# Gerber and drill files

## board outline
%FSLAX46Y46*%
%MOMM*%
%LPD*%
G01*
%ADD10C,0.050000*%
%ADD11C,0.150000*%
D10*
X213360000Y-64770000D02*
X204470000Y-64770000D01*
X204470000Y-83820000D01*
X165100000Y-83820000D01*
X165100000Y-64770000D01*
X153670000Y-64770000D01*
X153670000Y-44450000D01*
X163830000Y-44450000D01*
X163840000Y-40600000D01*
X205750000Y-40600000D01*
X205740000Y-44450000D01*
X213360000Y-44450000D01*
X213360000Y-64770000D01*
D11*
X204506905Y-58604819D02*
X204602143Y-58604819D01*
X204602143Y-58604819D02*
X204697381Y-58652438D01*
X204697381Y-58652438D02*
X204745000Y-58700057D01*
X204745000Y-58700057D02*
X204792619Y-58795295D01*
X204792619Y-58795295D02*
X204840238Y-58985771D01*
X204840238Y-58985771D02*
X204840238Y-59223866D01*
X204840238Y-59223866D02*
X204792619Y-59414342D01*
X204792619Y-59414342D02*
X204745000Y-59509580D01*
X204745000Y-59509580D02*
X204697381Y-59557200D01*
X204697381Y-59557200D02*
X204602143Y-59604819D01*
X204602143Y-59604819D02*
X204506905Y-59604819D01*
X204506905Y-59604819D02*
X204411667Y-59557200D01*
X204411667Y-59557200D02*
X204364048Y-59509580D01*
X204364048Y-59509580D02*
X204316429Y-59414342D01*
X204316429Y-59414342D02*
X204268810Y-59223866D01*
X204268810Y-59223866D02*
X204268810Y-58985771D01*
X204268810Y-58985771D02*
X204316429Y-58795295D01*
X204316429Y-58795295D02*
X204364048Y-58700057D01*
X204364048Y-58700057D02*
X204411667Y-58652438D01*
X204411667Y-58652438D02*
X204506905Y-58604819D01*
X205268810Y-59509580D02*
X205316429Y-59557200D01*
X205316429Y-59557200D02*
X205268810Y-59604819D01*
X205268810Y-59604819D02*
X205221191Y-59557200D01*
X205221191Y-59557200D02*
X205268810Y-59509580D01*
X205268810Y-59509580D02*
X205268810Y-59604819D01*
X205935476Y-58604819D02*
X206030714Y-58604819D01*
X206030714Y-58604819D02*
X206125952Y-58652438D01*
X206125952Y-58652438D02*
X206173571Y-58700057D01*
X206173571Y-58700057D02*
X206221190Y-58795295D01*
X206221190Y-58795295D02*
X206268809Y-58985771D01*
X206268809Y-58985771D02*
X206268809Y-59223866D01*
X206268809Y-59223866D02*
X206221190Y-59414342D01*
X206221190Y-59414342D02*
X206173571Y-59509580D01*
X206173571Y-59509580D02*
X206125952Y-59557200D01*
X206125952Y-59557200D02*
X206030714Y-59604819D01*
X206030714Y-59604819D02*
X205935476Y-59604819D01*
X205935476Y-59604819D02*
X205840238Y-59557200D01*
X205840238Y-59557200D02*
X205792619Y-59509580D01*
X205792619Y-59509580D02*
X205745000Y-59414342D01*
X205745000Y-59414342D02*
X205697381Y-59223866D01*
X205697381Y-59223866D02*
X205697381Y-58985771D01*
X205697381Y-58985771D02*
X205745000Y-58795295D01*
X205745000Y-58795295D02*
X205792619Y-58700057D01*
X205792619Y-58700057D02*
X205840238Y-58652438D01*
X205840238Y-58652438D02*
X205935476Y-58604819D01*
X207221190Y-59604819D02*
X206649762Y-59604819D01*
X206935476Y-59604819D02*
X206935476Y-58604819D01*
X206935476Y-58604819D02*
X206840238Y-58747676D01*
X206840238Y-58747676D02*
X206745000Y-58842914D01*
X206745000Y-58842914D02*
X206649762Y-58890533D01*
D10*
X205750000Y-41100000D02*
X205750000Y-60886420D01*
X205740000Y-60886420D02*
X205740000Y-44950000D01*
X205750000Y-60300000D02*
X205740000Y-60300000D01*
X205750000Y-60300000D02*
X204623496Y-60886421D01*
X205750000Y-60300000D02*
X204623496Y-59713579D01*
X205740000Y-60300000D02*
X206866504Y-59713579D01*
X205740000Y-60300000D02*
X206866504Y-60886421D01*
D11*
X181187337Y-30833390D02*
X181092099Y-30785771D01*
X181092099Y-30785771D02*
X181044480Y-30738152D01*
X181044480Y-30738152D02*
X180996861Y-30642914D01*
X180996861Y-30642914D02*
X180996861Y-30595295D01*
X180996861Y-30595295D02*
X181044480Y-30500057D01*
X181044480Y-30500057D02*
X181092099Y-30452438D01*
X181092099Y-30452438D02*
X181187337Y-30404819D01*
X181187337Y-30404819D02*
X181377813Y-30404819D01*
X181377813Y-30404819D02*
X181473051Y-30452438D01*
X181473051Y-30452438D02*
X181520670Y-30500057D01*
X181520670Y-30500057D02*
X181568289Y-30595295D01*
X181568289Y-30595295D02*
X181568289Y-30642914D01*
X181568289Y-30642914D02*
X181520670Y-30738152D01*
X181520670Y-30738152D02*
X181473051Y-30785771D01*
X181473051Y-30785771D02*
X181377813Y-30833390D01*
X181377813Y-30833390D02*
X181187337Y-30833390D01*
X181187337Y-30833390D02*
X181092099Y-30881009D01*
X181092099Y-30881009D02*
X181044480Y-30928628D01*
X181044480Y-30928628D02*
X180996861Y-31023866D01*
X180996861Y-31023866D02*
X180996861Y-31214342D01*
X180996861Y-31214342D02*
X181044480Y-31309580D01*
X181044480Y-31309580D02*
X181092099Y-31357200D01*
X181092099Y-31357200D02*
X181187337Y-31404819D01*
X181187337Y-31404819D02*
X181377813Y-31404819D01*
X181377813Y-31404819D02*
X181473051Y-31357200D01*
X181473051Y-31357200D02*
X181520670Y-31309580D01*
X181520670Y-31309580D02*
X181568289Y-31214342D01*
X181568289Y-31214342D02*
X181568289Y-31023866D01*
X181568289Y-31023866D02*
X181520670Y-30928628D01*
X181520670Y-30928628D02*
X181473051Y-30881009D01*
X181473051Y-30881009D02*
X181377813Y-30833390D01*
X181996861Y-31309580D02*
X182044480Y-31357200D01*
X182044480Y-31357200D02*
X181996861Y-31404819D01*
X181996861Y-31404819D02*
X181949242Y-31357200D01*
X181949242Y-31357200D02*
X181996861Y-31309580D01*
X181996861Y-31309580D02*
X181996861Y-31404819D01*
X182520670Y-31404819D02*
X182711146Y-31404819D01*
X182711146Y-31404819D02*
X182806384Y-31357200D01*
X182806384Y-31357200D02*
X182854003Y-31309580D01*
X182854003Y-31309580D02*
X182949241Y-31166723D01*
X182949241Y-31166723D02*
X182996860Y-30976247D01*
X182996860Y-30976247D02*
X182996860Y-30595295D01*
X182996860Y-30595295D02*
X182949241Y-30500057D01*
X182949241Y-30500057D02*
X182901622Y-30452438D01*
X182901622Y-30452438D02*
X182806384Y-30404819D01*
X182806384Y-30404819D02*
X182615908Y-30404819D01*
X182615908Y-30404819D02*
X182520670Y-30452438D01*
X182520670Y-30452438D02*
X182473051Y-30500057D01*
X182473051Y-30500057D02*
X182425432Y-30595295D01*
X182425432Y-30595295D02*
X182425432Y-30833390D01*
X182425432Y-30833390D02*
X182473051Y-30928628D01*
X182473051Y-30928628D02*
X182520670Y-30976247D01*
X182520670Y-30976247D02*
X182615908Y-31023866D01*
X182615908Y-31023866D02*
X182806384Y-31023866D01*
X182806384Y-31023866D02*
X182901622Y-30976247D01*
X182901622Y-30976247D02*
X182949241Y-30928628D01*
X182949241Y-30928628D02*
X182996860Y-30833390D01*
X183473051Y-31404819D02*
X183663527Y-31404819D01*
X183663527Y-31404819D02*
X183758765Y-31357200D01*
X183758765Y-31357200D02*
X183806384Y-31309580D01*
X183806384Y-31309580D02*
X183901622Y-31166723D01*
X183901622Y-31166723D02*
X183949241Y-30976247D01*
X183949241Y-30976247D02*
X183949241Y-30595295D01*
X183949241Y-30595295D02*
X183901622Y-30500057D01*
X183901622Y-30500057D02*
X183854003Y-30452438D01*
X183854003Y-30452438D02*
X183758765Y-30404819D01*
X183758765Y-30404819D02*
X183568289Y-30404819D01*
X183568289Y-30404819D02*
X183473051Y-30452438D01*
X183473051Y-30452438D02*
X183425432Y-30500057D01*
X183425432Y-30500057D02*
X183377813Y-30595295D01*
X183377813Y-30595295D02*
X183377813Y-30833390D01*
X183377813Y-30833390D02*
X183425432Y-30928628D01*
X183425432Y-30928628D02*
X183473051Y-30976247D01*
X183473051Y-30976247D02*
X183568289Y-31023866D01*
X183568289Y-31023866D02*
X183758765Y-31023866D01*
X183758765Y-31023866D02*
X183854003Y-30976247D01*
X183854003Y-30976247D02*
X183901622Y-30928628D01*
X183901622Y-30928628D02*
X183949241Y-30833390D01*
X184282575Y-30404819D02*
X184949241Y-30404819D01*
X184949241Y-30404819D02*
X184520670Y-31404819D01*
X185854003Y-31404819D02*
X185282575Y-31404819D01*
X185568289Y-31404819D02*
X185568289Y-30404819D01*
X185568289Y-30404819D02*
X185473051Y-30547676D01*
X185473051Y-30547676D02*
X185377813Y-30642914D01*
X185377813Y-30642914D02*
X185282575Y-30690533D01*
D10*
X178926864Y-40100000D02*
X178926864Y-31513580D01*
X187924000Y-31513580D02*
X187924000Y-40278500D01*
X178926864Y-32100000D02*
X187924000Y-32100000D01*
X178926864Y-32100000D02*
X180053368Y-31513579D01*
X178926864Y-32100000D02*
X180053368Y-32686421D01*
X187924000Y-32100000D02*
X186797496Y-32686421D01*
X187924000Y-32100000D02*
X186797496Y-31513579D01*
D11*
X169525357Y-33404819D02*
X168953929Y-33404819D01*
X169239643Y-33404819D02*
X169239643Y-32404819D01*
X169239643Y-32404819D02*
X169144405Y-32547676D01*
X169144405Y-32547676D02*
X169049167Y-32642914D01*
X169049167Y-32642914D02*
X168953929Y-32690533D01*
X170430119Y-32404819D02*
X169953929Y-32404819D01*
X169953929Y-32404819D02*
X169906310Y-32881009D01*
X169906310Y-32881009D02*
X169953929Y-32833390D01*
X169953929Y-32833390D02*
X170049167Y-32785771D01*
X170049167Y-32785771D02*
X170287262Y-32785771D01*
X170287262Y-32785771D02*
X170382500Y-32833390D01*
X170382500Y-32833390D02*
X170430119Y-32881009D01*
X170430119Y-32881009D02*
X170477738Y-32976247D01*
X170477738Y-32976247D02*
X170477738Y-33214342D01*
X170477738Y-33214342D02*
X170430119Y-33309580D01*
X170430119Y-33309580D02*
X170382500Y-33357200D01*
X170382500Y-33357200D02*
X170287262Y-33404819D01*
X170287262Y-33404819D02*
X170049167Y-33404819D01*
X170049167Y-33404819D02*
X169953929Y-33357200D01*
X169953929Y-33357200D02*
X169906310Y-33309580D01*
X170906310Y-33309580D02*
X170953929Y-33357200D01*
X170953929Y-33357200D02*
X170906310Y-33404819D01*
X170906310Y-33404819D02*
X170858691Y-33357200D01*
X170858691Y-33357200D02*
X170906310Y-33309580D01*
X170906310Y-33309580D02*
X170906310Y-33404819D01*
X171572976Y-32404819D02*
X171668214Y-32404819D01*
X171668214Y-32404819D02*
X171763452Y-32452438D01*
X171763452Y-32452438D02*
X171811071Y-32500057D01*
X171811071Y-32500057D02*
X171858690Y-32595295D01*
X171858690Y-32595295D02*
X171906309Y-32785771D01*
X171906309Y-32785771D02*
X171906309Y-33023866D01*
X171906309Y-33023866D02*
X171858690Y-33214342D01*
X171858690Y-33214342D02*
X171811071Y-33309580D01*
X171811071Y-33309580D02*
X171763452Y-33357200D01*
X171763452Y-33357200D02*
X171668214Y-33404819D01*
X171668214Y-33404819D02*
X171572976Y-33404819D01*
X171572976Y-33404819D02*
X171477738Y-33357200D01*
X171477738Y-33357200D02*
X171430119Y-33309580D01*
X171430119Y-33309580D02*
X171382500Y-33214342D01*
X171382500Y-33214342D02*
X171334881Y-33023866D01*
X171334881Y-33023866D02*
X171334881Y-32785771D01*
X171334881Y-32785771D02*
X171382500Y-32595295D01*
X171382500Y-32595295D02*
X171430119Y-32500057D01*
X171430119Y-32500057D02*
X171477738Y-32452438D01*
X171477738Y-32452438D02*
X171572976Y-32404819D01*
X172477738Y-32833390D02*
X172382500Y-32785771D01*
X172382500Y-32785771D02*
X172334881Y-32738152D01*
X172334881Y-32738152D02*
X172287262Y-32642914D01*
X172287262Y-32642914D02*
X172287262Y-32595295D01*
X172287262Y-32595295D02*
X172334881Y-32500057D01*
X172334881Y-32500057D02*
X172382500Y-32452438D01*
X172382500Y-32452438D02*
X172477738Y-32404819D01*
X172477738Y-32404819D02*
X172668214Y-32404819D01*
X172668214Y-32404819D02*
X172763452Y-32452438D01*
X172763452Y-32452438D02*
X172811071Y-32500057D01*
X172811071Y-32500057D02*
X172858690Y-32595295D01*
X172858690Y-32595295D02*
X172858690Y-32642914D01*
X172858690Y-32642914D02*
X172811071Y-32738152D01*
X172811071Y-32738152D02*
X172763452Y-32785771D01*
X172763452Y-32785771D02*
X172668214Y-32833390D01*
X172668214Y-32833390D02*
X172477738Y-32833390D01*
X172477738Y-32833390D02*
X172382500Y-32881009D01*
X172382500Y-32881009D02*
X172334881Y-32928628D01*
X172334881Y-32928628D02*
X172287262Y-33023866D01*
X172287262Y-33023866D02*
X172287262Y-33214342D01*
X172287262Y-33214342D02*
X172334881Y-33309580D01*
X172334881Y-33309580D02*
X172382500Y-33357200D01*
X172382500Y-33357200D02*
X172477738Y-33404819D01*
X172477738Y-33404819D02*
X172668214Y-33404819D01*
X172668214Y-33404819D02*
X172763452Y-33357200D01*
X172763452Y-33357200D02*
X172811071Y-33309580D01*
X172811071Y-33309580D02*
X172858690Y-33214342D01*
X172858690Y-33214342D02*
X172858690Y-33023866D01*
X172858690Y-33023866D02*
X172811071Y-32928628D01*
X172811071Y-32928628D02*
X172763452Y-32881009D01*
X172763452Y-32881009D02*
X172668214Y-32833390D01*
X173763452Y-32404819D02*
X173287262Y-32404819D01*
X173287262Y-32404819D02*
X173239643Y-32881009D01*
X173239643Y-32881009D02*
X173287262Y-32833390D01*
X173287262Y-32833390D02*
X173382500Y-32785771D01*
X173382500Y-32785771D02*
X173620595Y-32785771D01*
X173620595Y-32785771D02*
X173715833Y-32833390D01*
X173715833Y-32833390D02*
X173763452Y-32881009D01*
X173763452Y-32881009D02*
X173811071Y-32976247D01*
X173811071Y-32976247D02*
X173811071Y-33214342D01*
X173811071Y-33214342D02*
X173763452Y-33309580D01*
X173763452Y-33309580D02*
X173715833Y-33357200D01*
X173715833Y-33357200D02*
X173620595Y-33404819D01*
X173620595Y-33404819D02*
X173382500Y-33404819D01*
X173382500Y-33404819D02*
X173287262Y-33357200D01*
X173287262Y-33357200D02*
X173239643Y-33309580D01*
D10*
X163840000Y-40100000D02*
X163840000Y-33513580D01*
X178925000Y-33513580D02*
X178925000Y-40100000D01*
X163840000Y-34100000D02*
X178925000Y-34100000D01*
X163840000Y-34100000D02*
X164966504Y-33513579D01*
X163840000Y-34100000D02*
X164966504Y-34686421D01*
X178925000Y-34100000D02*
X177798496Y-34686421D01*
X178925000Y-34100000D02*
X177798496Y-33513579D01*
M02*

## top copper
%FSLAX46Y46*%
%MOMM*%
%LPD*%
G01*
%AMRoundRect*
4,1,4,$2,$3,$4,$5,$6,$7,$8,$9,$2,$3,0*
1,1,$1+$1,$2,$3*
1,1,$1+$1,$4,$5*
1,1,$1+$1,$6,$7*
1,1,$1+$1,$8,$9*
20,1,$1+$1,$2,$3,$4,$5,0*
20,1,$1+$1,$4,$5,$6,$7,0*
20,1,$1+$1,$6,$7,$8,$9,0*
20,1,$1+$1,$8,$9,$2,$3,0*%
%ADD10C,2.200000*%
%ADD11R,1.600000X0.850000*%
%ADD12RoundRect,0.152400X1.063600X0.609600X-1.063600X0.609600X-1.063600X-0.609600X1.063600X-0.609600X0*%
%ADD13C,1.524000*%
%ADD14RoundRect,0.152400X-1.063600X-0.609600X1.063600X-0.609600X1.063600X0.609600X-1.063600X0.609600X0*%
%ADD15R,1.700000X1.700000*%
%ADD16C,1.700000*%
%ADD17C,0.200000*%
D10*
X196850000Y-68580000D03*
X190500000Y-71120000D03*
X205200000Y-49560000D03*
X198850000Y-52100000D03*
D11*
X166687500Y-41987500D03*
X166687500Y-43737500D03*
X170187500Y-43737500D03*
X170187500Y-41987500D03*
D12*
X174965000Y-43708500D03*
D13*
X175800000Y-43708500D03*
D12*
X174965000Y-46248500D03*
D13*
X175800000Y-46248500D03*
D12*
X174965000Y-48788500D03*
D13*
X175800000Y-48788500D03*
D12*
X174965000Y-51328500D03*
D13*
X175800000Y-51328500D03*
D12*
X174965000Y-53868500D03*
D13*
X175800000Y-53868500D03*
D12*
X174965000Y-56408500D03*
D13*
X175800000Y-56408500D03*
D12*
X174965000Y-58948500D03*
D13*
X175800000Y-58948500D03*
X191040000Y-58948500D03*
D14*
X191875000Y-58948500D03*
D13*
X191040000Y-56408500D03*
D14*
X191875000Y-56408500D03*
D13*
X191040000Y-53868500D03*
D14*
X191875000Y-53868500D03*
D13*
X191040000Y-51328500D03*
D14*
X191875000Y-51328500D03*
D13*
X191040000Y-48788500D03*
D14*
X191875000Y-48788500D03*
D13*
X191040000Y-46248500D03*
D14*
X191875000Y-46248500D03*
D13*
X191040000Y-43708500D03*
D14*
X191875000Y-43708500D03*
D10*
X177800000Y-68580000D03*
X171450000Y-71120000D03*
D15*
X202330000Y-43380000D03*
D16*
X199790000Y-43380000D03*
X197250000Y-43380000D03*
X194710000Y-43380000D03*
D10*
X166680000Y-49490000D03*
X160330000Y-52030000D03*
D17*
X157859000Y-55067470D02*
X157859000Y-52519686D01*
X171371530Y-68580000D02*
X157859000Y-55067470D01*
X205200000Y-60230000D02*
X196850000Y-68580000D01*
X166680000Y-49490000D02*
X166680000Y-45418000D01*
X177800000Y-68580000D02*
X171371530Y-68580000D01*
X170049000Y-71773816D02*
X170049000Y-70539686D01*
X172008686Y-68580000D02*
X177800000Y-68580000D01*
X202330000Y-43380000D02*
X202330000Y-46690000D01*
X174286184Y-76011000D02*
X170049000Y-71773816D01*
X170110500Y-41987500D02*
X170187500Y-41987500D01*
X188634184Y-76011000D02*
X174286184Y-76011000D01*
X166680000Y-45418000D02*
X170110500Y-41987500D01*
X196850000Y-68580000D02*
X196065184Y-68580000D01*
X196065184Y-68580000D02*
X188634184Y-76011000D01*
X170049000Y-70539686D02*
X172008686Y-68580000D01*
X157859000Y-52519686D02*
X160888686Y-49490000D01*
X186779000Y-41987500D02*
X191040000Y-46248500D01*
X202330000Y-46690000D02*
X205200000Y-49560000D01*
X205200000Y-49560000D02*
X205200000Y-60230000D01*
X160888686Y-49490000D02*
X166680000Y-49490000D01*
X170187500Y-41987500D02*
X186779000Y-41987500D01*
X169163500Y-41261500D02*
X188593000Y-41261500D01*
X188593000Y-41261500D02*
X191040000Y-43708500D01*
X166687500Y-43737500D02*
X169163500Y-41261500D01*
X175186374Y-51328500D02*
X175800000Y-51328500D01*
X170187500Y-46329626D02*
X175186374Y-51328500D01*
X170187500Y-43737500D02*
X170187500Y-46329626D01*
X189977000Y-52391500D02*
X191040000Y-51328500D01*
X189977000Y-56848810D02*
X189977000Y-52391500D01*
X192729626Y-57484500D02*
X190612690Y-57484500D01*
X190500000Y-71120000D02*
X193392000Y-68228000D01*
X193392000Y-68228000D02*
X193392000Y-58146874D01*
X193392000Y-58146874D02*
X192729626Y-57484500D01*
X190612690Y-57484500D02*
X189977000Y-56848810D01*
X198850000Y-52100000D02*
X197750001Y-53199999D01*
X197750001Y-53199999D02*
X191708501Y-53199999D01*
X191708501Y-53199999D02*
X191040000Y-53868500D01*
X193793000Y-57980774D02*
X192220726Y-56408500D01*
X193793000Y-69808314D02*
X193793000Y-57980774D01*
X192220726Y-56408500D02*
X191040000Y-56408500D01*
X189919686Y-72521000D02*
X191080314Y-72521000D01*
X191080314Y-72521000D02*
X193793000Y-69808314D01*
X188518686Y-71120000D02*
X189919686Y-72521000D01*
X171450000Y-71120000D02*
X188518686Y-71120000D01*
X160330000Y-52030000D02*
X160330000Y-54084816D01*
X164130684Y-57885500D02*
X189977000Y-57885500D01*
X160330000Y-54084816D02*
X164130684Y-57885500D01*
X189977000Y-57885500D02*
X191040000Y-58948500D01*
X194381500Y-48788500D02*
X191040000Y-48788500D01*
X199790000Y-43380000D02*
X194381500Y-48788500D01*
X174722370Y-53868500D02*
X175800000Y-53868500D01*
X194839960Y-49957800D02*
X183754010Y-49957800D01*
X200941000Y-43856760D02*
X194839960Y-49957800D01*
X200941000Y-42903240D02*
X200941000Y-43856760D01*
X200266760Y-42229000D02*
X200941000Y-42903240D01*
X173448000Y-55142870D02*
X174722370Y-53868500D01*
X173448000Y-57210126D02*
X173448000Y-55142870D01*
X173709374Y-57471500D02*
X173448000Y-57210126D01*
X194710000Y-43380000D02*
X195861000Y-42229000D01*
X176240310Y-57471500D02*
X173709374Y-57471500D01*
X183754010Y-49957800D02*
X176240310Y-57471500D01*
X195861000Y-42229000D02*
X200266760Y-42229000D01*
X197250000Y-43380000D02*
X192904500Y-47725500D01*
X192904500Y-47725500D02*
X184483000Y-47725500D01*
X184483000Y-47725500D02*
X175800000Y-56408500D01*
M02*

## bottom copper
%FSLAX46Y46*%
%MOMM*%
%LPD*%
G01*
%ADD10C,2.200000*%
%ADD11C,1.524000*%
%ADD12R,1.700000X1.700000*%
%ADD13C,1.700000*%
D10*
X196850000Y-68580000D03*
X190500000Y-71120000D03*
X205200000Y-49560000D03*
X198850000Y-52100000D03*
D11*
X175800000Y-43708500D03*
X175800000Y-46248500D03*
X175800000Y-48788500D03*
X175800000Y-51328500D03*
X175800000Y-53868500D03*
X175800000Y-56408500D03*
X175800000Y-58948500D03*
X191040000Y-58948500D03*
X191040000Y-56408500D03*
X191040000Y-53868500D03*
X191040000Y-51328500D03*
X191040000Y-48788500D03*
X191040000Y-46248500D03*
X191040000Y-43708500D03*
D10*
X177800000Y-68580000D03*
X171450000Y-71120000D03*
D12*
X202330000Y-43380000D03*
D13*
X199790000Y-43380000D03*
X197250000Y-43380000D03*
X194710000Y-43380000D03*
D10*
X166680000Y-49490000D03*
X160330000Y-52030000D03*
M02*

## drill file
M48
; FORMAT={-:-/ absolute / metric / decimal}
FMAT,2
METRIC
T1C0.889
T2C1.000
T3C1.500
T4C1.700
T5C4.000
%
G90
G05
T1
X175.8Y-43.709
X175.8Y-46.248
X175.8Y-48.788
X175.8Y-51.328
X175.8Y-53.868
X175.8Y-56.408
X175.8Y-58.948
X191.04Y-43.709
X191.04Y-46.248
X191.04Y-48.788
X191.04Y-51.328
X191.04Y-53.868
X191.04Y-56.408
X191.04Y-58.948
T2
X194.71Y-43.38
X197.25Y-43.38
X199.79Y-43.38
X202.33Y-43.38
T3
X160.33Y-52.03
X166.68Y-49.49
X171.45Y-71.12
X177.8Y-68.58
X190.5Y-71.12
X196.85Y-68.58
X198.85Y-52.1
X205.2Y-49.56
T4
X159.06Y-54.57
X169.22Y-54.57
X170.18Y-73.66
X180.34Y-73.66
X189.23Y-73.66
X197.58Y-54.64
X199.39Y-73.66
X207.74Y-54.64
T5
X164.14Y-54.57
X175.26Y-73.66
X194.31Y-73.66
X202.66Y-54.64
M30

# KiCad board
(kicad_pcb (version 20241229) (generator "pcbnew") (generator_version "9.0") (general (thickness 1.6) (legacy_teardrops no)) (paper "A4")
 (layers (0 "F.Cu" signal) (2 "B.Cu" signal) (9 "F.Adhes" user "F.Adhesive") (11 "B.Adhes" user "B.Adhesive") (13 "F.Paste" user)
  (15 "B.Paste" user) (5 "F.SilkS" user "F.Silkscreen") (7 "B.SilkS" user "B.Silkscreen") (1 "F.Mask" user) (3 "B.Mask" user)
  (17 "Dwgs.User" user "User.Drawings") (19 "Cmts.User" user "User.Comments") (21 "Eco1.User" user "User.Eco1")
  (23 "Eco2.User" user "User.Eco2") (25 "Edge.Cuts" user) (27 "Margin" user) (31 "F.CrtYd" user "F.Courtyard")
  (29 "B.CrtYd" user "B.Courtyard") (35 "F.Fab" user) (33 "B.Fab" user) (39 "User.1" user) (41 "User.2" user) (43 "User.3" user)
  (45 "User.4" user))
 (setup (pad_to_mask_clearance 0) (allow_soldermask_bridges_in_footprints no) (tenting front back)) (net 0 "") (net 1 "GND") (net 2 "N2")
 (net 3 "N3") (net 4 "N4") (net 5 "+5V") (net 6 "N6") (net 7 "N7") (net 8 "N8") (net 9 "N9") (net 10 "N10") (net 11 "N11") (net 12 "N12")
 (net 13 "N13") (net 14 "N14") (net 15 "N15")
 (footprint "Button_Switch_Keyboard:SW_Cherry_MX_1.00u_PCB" (layer "F.Cu") (at 196.85 68.58)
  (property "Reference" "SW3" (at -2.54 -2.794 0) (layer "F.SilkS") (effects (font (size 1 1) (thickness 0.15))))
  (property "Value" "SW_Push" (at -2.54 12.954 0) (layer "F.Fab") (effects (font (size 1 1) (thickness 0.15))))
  (pad "" np_thru_hole circle (at -7.62 5.08) (size 1.7 1.7) (drill 1.7) (layers "*.Cu" "*.Mask"))
  (pad "" np_thru_hole circle (at -2.54 5.08) (size 4 4) (drill 4) (layers "*.Cu" "*.Mask"))
  (pad "" np_thru_hole circle (at 2.54 5.08) (size 1.7 1.7) (drill 1.7) (layers "*.Cu" "*.Mask"))
  (pad "1" thru_hole circle (at 0 0) (size 2.2 2.2) (drill 1.5) (layers "*.Cu" "*.Mask") (remove_unused_layers no) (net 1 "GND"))
  (pad "2" thru_hole circle (at -6.35 2.54) (size 2.2 2.2) (drill 1.5) (layers "*.Cu" "*.Mask") (remove_unused_layers no) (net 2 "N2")))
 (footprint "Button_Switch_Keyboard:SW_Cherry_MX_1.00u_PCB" (layer "F.Cu") (at 205.2 49.56)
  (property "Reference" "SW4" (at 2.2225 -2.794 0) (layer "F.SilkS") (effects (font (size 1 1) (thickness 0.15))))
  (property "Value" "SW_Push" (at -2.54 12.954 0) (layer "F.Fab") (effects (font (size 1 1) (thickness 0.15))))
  (pad "" np_thru_hole circle (at -7.62 5.08) (size 1.7 1.7) (drill 1.7) (layers "*.Cu" "*.Mask"))
  (pad "" np_thru_hole circle (at -2.54 5.08) (size 4 4) (drill 4) (layers "*.Cu" "*.Mask"))
  (pad "" np_thru_hole circle (at 2.54 5.08) (size 1.7 1.7) (drill 1.7) (layers "*.Cu" "*.Mask"))
  (pad "1" thru_hole circle (at 0 0) (size 2.2 2.2) (drill 1.5) (layers "*.Cu" "*.Mask") (remove_unused_layers no) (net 1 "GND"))
  (pad "2" thru_hole circle (at -6.35 2.54) (size 2.2 2.2) (drill 1.5) (layers "*.Cu" "*.Mask") (remove_unused_layers no) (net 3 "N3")))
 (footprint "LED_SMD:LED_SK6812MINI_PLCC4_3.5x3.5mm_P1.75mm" (layer "F.Cu") (at 168.4375 42.8625)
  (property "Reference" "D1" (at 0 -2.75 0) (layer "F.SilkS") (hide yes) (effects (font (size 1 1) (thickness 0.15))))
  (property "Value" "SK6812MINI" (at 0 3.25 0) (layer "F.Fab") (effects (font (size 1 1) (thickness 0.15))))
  (pad "1" smd rect (at -1.75 -0.875) (size 1.6 0.85) (layers "F.Cu" "F.Mask" "F.Paste") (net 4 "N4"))
  (pad "2" smd rect (at -1.75 0.875) (size 1.6 0.85) (layers "F.Cu" "F.Mask" "F.Paste") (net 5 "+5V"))
  (pad "3" smd rect (at 1.75 0.875) (size 1.6 0.85) (layers "F.Cu" "F.Mask" "F.Paste") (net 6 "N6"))
  (pad "4" smd rect (at 1.75 -0.875) (size 1.6 0.85) (layers "F.Cu" "F.Mask" "F.Paste") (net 1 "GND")))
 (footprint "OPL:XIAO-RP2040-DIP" (layer "F.Cu") (at 183.42 51.3285)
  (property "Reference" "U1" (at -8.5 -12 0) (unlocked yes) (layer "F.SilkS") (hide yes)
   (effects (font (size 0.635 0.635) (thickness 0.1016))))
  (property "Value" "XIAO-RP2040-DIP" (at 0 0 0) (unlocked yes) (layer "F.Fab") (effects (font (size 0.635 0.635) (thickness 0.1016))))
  (pad "1" smd roundrect (at -8.455 -7.62 180) (size 2.432 1.524) (layers "F.Cu" "F.Mask") (roundrect_rratio 0.1) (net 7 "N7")
   (thermal_bridge_angle 45))
  (pad "1" thru_hole circle (at -7.62 -7.62 180) (size 1.524 1.524) (drill 0.889) (layers "*.Cu" "*.Mask") (remove_unused_layers no)
   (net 7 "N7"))
  (pad "2" smd roundrect (at -8.455 -5.08 180) (size 2.432 1.524) (layers "F.Cu" "F.Mask") (roundrect_rratio 0.1) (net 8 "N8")
   (thermal_bridge_angle 45))
  (pad "2" thru_hole circle (at -7.62 -5.08 180) (size 1.524 1.524) (drill 0.889) (layers "*.Cu" "*.Mask") (remove_unused_layers no)
   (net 8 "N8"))
  (pad "3" smd roundrect (at -8.455 -2.54 180) (size 2.432 1.524) (layers "F.Cu" "F.Mask") (roundrect_rratio 0.1) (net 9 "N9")
   (thermal_bridge_angle 45))
  (pad "3" thru_hole circle (at -7.62 -2.54 180) (size 1.524 1.524) (drill 0.889) (layers "*.Cu" "*.Mask") (remove_unused_layers no)
   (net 9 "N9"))
  (pad "4" smd roundrect (at -8.455 0 180) (size 2.432 1.524) (layers "F.Cu" "F.Mask") (roundrect_rratio 0.1) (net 6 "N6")
   (thermal_bridge_angle 45))
  (pad "4" thru_hole circle (at -7.62 0 180) (size 1.524 1.524) (drill 0.889) (layers "*.Cu" "*.Mask") (remove_unused_layers no)
   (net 6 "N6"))
  (pad "5" smd roundrect (at -8.455 2.54 180) (size 2.432 1.524) (layers "F.Cu" "F.Mask") (roundrect_rratio 0.1) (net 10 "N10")
   (thermal_bridge_angle 45))
  (pad "5" thru_hole circle (at -7.62 2.54 180) (size 1.524 1.524) (drill 0.889) (layers "*.Cu" "*.Mask") (remove_unused_layers no)
   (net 10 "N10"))
  (pad "6" smd roundrect (at -8.455 5.08 180) (size 2.432 1.524) (layers "F.Cu" "F.Mask") (roundrect_rratio 0.1) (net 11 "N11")
   (thermal_bridge_angle 45))
  (pad "6" thru_hole circle (at -7.62 5.08 180) (size 1.524 1.524) (drill 0.889) (layers "*.Cu" "*.Mask") (remove_unused_layers no)
   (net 11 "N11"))
  (pad "7" smd roundrect (at -8.455 7.62 180) (size 2.432 1.524) (layers "F.Cu" "F.Mask") (roundrect_rratio 0.1) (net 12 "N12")
   (thermal_bridge_angle 45))
  (pad "7" thru_hole circle (at -7.62 7.62 180) (size 1.524 1.524) (drill 0.889) (layers "*.Cu" "*.Mask") (remove_unused_layers no)
   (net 12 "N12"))
  (pad "8" thru_hole circle (at 7.62 7.62) (size 1.524 1.524) (drill 0.889) (layers "*.Cu" "*.Mask") (remove_unused_layers no)
   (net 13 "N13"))
  (pad "8" smd roundrect (at 8.455 7.62) (size 2.432 1.524) (layers "F.Cu" "F.Mask") (roundrect_rratio 0.1) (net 13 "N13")
   (thermal_bridge_angle 45))
  (pad "9" thru_hole circle (at 7.62 5.08) (size 1.524 1.524) (drill 0.889) (layers "*.Cu" "*.Mask") (remove_unused_layers no)
   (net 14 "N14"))
  (pad "9" smd roundrect (at 8.455 5.08) (size 2.432 1.524) (layers "F.Cu" "F.Mask") (roundrect_rratio 0.1) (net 14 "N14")
   (thermal_bridge_angle 45))
  (pad "10" thru_hole circle (at 7.62 2.54) (size 1.524 1.524) (drill 0.889) (layers "*.Cu" "*.Mask") (remove_unused_layers no) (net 3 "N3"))
  (pad "10" smd roundrect (at 8.455 2.54) (size 2.432 1.524) (layers "F.Cu" "F.Mask") (roundrect_rratio 0.1) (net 3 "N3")
   (thermal_bridge_angle 45))
  (pad "11" thru_hole circle (at 7.62 0) (size 1.524 1.524) (drill 0.889) (layers "*.Cu" "*.Mask") (remove_unused_layers no) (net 2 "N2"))
  (pad "11" smd roundrect (at 8.455 0) (size 2.432 1.524) (layers "F.Cu" "F.Mask") (roundrect_rratio 0.1) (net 2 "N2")
   (thermal_bridge_angle 45))
  (pad "12" thru_hole circle (at 7.62 -2.54) (size 1.524 1.524) (drill 0.889) (layers "*.Cu" "*.Mask") (remove_unused_layers no)
   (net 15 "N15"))
  (pad "12" smd roundrect (at 8.455 -2.54) (size 2.432 1.524) (layers "F.Cu" "F.Mask") (roundrect_rratio 0.1) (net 15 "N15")
   (thermal_bridge_angle 45))
  (pad "13" thru_hole circle (at 7.62 -5.08) (size 1.524 1.524) (drill 0.889) (layers "*.Cu" "*.Mask") (remove_unused_layers no)
   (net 1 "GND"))
  (pad "13" smd roundrect (at 8.455 -5.08) (size 2.432 1.524) (layers "F.Cu" "F.Mask") (roundrect_rratio 0.1) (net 1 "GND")
   (thermal_bridge_angle 45))
  (pad "14" thru_hole circle (at 7.62 -7.62) (size 1.524 1.524) (drill 0.889) (layers "*.Cu" "*.Mask") (remove_unused_layers no)
   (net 5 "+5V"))
  (pad "14" smd roundrect (at 8.455 -7.62) (size 2.432 1.524) (layers "F.Cu" "F.Mask") (roundrect_rratio 0.1) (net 5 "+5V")
   (thermal_bridge_angle 45)))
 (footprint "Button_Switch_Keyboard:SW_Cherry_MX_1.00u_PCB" (layer "F.Cu") (at 177.8 68.58)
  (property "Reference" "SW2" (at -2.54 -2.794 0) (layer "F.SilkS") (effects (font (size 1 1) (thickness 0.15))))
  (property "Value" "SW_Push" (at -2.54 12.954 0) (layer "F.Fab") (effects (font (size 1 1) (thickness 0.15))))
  (pad "" np_thru_hole circle (at -7.62 5.08) (size 1.7 1.7) (drill 1.7) (layers "*.Cu" "*.Mask"))
  (pad "" np_thru_hole circle (at -2.54 5.08) (size 4 4) (drill 4) (layers "*.Cu" "*.Mask"))
  (pad "" np_thru_hole circle (at 2.54 5.08) (size 1.7 1.7) (drill 1.7) (layers "*.Cu" "*.Mask"))
  (pad "1" thru_hole circle (at 0 0) (size 2.2 2.2) (drill 1.5) (layers "*.Cu" "*.Mask") (remove_unused_layers no) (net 1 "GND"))
  (pad "2" thru_hole circle (at -6.35 2.54) (size 2.2 2.2) (drill 1.5) (layers "*.Cu" "*.Mask") (remove_unused_layers no) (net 14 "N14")))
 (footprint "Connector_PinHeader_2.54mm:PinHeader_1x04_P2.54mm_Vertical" (layer "F.Cu") (at 202.33 43.38 -90)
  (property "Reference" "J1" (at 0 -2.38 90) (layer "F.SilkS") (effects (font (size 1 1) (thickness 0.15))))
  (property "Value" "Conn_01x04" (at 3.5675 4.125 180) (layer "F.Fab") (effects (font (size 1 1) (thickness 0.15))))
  (pad "1" thru_hole rect (at 0 0 270) (size 1.7 1.7) (drill 1) (layers "*.Cu" "*.Mask") (remove_unused_layers no) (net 1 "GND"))
  (pad "2" thru_hole circle (at 0 2.54 270) (size 1.7 1.7) (drill 1) (layers "*.Cu" "*.Mask") (remove_unused_layers no) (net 15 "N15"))
  (pad "3" thru_hole circle (at 0 5.08 270) (size 1.7 1.7) (drill 1) (layers "*.Cu" "*.Mask") (remove_unused_layers no) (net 11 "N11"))
  (pad "4" thru_hole circle (at 0 7.62 270) (size 1.7 1.7) (drill 1) (layers "*.Cu" "*.Mask") (remove_unused_layers no) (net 10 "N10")))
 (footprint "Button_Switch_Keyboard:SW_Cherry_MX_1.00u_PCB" (layer "F.Cu") (at 166.68 49.49)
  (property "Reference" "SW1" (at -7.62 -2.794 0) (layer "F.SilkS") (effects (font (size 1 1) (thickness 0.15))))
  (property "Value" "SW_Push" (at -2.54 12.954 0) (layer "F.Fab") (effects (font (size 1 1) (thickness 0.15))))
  (pad "" np_thru_hole circle (at -7.62 5.08) (size 1.7 1.7) (drill 1.7) (layers "*.Cu" "*.Mask"))
  (pad "" np_thru_hole circle (at -2.54 5.08) (size 4 4) (drill 4) (layers "*.Cu" "*.Mask"))
  (pad "" np_thru_hole circle (at 2.54 5.08) (size 1.7 1.7) (drill 1.7) (layers "*.Cu" "*.Mask"))
  (pad "1" thru_hole circle (at 0 0) (size 2.2 2.2) (drill 1.5) (layers "*.Cu" "*.Mask") (remove_unused_layers no) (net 1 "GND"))
  (pad "2" thru_hole circle (at -6.35 2.54) (size 2.2 2.2) (drill 1.5) (layers "*.Cu" "*.Mask") (remove_unused_layers no) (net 13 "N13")))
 (gr_poly
  (pts (xy 213.36 64.77) (xy 204.47 64.77) (xy 204.47 83.82) (xy 165.1 83.82) (xy 165.1 64.77) (xy 153.67 64.77) (xy 153.67 44.45)
   (xy 163.83 44.45) (xy 163.84 40.6) (xy 205.75 40.6) (xy 205.74 44.45) (xy 213.36 44.45))
  (stroke (width 0.05) (type solid)) (fill no) (layer "Edge.Cuts"))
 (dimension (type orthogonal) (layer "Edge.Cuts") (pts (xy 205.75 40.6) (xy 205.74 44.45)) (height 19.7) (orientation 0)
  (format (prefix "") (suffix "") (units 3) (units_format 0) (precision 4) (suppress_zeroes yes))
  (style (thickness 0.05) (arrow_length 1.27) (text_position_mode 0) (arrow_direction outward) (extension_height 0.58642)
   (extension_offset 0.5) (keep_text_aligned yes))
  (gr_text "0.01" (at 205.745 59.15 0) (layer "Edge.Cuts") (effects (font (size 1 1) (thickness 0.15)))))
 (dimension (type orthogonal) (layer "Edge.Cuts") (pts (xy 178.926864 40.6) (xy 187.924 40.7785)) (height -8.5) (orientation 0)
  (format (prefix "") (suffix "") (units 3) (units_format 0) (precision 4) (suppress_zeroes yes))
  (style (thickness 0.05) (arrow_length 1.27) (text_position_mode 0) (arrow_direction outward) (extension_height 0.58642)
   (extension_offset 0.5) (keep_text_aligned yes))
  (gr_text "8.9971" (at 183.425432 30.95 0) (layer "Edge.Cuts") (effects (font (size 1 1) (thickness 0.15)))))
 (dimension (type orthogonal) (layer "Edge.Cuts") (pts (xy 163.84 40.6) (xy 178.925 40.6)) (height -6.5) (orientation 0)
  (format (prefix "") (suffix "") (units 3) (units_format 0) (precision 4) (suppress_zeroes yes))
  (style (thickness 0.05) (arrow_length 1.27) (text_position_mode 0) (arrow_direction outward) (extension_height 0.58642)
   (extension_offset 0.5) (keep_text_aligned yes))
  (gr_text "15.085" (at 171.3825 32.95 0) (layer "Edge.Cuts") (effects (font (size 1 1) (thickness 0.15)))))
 (segment (start 157.859 55.06747) (end 157.859 52.519686) (width 0.2) (layer "F.Cu") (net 1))
 (segment (start 171.37153 68.58) (end 157.859 55.06747) (width 0.2) (layer "F.Cu") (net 1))
 (segment (start 205.2 60.23) (end 196.85 68.58) (width 0.2) (layer "F.Cu") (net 1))
 (segment (start 166.68 49.49) (end 166.68 45.418) (width 0.2) (layer "F.Cu") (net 1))
 (segment (start 177.8 68.58) (end 171.37153 68.58) (width 0.2) (layer "F.Cu") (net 1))
 (segment (start 170.049 71.773816) (end 170.049 70.539686) (width 0.2) (layer "F.Cu") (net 1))
 (segment (start 172.008686 68.58) (end 177.8 68.58) (width 0.2) (layer "F.Cu") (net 1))
 (segment (start 202.33 43.38) (end 202.33 46.69) (width 0.2) (layer "F.Cu") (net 1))
 (segment (start 174.286184 76.011) (end 170.049 71.773816) (width 0.2) (layer "F.Cu") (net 1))
 (segment (start 170.1105 41.9875) (end 170.1875 41.9875) (width 0.2) (layer "F.Cu") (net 1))
 (segment (start 188.634184 76.011) (end 174.286184 76.011) (width 0.2) (layer "F.Cu") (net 1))
 (segment (start 166.68 45.418) (end 170.1105 41.9875) (width 0.2) (layer "F.Cu") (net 1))
 (segment (start 196.85 68.58) (end 196.065184 68.58) (width 0.2) (layer "F.Cu") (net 1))
 (segment (start 196.065184 68.58) (end 188.634184 76.011) (width 0.2) (layer "F.Cu") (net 1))
 (segment (start 170.049 70.539686) (end 172.008686 68.58) (width 0.2) (layer "F.Cu") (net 1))
 (segment (start 157.859 52.519686) (end 160.888686 49.49) (width 0.2) (layer "F.Cu") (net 1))
 (segment (start 186.779 41.9875) (end 191.04 46.2485) (width 0.2) (layer "F.Cu") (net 1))
 (segment (start 202.33 46.69) (end 205.2 49.56) (width 0.2) (layer "F.Cu") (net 1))
 (segment (start 205.2 49.56) (end 205.2 60.23) (width 0.2) (layer "F.Cu") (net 1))
 (segment (start 160.888686 49.49) (end 166.68 49.49) (width 0.2) (layer "F.Cu") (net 1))
 (segment (start 170.1875 41.9875) (end 186.779 41.9875) (width 0.2) (layer "F.Cu") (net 1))
 (segment (start 169.1635 41.2615) (end 188.593 41.2615) (width 0.2) (layer "F.Cu") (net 5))
 (segment (start 188.593 41.2615) (end 191.04 43.7085) (width 0.2) (layer "F.Cu") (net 5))
 (segment (start 166.6875 43.7375) (end 169.1635 41.2615) (width 0.2) (layer "F.Cu") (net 5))
 (segment (start 175.186374 51.3285) (end 175.8 51.3285) (width 0.2) (layer "F.Cu") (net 6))
 (segment (start 170.1875 46.329626) (end 175.186374 51.3285) (width 0.2) (layer "F.Cu") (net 6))
 (segment (start 170.1875 43.7375) (end 170.1875 46.329626) (width 0.2) (layer "F.Cu") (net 6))
 (segment (start 189.977 52.3915) (end 191.04 51.3285) (width 0.2) (layer "F.Cu") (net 2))
 (segment (start 189.977 56.84881) (end 189.977 52.3915) (width 0.2) (layer "F.Cu") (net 2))
 (segment (start 192.729626 57.4845) (end 190.61269 57.4845) (width 0.2) (layer "F.Cu") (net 2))
 (segment (start 190.5 71.12) (end 193.392 68.228) (width 0.2) (layer "F.Cu") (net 2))
 (segment (start 193.392 68.228) (end 193.392 58.146874) (width 0.2) (layer "F.Cu") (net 2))
 (segment (start 193.392 58.146874) (end 192.729626 57.4845) (width 0.2) (layer "F.Cu") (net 2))
 (segment (start 190.61269 57.4845) (end 189.977 56.84881) (width 0.2) (layer "F.Cu") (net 2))
 (segment (start 198.85 52.1) (end 197.750001 53.199999) (width 0.2) (layer "F.Cu") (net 3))
 (segment (start 197.750001 53.199999) (end 191.708501 53.199999) (width 0.2) (layer "F.Cu") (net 3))
 (segment (start 191.708501 53.199999) (end 191.04 53.8685) (width 0.2) (layer "F.Cu") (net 3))
 (segment (start 193.793 57.980774) (end 192.220726 56.4085) (width 0.2) (layer "F.Cu") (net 14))
 (segment (start 193.793 69.808314) (end 193.793 57.980774) (width 0.2) (layer "F.Cu") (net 14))
 (segment (start 192.220726 56.4085) (end 191.04 56.4085) (width 0.2) (layer "F.Cu") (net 14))
 (segment (start 189.919686 72.521) (end 191.080314 72.521) (width 0.2) (layer "F.Cu") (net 14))
 (segment (start 191.080314 72.521) (end 193.793 69.808314) (width 0.2) (layer "F.Cu") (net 14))
 (segment (start 188.518686 71.12) (end 189.919686 72.521) (width 0.2) (layer "F.Cu") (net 14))
 (segment (start 171.45 71.12) (end 188.518686 71.12) (width 0.2) (layer "F.Cu") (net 14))
 (segment (start 160.33 52.03) (end 160.33 54.084816) (width 0.2) (layer "F.Cu") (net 13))
 (segment (start 164.130684 57.8855) (end 189.977 57.8855) (width 0.2) (layer "F.Cu") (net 13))
 (segment (start 160.33 54.084816) (end 164.130684 57.8855) (width 0.2) (layer "F.Cu") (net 13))
 (segment (start 189.977 57.8855) (end 191.04 58.9485) (width 0.2) (layer "F.Cu") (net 13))
 (segment (start 194.3815 48.7885) (end 191.04 48.7885) (width 0.2) (layer "F.Cu") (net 15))
 (segment (start 199.79 43.38) (end 194.3815 48.7885) (width 0.2) (layer "F.Cu") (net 15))
 (segment (start 174.72237 53.8685) (end 175.8 53.8685) (width 0.2) (layer "F.Cu") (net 10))
 (segment (start 194.83996 49.9578) (end 183.75401 49.9578) (width 0.2) (layer "F.Cu") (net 10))
 (segment (start 200.941 43.85676) (end 194.83996 49.9578) (width 0.2) (layer "F.Cu") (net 10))
 (segment (start 200.941 42.90324) (end 200.941 43.85676) (width 0.2) (layer "F.Cu") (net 10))
 (segment (start 200.26676 42.229) (end 200.941 42.90324) (width 0.2) (layer "F.Cu") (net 10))
 (segment (start 173.448 55.14287) (end 174.72237 53.8685) (width 0.2) (layer "F.Cu") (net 10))
 (segment (start 173.448 57.210126) (end 173.448 55.14287) (width 0.2) (layer "F.Cu") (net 10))
 (segment (start 173.709374 57.4715) (end 173.448 57.210126) (width 0.2) (layer "F.Cu") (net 10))
 (segment (start 194.71 43.38) (end 195.861 42.229) (width 0.2) (layer "F.Cu") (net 10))
 (segment (start 176.24031 57.4715) (end 173.709374 57.4715) (width 0.2) (layer "F.Cu") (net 10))
 (segment (start 183.75401 49.9578) (end 176.24031 57.4715) (width 0.2) (layer "F.Cu") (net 10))
 (segment (start 195.861 42.229) (end 200.26676 42.229) (width 0.2) (layer "F.Cu") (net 10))
 (segment (start 197.25 43.38) (end 192.9045 47.7255) (width 0.2) (layer "F.Cu") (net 11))
 (segment (start 192.9045 47.7255) (end 184.483 47.7255) (width 0.2) (layer "F.Cu") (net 11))
 (segment (start 184.483 47.7255) (end 175.8 56.4085) (width 0.2) (layer "F.Cu") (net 11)))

